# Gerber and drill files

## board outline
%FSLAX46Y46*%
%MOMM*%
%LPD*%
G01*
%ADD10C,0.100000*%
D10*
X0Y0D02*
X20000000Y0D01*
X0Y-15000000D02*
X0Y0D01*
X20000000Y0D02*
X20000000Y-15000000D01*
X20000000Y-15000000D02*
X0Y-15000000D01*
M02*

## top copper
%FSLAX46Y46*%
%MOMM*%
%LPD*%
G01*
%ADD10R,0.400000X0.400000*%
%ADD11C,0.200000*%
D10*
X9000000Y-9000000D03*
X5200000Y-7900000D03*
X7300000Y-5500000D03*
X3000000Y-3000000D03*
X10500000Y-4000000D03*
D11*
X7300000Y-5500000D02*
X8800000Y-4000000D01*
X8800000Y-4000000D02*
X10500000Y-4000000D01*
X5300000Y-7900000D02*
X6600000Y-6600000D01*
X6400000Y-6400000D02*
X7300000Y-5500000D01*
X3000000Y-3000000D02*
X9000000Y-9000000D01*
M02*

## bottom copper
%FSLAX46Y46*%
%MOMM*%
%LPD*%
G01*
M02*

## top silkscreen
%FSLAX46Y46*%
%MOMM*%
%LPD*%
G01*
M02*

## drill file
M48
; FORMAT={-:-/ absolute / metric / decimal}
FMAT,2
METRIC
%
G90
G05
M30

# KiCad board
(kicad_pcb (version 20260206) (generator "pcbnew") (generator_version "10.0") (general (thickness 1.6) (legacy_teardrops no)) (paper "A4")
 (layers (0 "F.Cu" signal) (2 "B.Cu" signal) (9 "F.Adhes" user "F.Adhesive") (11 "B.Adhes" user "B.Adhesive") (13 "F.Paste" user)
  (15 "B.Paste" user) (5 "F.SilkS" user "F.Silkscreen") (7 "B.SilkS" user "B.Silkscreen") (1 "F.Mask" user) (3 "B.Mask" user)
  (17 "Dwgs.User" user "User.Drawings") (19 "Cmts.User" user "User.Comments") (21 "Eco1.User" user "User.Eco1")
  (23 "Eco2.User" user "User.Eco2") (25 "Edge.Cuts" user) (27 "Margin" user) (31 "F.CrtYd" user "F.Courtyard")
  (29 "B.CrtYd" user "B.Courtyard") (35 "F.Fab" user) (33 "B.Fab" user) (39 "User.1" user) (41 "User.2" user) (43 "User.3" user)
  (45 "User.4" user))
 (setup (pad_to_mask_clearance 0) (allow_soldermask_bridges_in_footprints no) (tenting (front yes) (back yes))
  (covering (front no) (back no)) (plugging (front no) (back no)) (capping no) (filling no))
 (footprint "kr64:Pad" (layer "F.Cu") (at 9 9)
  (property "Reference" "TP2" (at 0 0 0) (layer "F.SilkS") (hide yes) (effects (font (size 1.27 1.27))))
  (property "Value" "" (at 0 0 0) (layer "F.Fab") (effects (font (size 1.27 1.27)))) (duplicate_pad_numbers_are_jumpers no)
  (pad "1" smd rect (at 0 0) (size 0.4 0.4) (layers "F.Cu" "F.Mask" "F.Paste") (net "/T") (thermal_bridge_angle 45)))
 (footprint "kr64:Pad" (layer "F.Cu") (at 5.2 7.9)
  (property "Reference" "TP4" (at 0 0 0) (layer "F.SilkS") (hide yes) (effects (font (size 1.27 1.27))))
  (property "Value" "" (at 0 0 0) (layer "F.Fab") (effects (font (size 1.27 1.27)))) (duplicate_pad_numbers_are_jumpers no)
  (pad "1" smd rect (at 0 0) (size 0.4 0.4) (layers "F.Cu" "F.Mask" "F.Paste") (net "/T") (thermal_bridge_angle 45)))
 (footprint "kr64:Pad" (layer "F.Cu") (at 7.3 5.5)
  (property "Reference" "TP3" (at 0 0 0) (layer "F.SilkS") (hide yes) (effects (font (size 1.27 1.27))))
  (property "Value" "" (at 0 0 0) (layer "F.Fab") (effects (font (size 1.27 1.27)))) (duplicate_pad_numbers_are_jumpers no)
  (pad "1" smd rect (at 0 0) (size 0.4 0.4) (layers "F.Cu" "F.Mask" "F.Paste") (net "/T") (thermal_bridge_angle 45)))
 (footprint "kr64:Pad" (layer "F.Cu") (at 3 3)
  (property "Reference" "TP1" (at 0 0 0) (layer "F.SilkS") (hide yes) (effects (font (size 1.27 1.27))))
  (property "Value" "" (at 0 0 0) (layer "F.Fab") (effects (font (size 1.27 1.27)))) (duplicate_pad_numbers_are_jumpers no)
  (pad "1" smd rect (at 0 0) (size 0.4 0.4) (layers "F.Cu" "F.Mask" "F.Paste") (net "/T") (thermal_bridge_angle 45)))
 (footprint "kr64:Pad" (layer "F.Cu") (at 10.5 4)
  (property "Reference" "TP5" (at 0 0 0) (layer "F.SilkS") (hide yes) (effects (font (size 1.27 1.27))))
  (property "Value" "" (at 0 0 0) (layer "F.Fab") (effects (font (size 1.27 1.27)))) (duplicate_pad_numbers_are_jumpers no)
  (pad "1" smd rect (at 0 0) (size 0.4 0.4) (layers "F.Cu" "F.Mask" "F.Paste") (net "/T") (thermal_bridge_angle 45)))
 (gr_line (start 0 0) (end 20 0) (stroke (width 0.1) (type default)) (layer "Edge.Cuts"))
 (gr_line (start 0 15) (end 0 0) (stroke (width 0.1) (type default)) (layer "Edge.Cuts"))
 (gr_line (start 20 0) (end 20 15) (stroke (width 0.1) (type default)) (layer "Edge.Cuts"))
 (gr_line (start 20 15) (end 0 15) (stroke (width 0.1) (type default)) (layer "Edge.Cuts"))
 (segment (start 7.3 5.5) (end 8.8 4) (width 0.2) (layer "F.Cu") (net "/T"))
 (segment (start 8.8 4) (end 10.5 4) (width 0.2) (layer "F.Cu") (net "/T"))
 (segment (start 5.3 7.9) (end 6.6 6.6) (width 0.2) (layer "F.Cu") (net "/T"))
 (segment (start 6.4 6.4) (end 7.3 5.5) (width 0.2) (layer "F.Cu") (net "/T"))
 (segment (start 3 3) (end 9 9) (width 0.2) (layer "F.Cu") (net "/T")))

